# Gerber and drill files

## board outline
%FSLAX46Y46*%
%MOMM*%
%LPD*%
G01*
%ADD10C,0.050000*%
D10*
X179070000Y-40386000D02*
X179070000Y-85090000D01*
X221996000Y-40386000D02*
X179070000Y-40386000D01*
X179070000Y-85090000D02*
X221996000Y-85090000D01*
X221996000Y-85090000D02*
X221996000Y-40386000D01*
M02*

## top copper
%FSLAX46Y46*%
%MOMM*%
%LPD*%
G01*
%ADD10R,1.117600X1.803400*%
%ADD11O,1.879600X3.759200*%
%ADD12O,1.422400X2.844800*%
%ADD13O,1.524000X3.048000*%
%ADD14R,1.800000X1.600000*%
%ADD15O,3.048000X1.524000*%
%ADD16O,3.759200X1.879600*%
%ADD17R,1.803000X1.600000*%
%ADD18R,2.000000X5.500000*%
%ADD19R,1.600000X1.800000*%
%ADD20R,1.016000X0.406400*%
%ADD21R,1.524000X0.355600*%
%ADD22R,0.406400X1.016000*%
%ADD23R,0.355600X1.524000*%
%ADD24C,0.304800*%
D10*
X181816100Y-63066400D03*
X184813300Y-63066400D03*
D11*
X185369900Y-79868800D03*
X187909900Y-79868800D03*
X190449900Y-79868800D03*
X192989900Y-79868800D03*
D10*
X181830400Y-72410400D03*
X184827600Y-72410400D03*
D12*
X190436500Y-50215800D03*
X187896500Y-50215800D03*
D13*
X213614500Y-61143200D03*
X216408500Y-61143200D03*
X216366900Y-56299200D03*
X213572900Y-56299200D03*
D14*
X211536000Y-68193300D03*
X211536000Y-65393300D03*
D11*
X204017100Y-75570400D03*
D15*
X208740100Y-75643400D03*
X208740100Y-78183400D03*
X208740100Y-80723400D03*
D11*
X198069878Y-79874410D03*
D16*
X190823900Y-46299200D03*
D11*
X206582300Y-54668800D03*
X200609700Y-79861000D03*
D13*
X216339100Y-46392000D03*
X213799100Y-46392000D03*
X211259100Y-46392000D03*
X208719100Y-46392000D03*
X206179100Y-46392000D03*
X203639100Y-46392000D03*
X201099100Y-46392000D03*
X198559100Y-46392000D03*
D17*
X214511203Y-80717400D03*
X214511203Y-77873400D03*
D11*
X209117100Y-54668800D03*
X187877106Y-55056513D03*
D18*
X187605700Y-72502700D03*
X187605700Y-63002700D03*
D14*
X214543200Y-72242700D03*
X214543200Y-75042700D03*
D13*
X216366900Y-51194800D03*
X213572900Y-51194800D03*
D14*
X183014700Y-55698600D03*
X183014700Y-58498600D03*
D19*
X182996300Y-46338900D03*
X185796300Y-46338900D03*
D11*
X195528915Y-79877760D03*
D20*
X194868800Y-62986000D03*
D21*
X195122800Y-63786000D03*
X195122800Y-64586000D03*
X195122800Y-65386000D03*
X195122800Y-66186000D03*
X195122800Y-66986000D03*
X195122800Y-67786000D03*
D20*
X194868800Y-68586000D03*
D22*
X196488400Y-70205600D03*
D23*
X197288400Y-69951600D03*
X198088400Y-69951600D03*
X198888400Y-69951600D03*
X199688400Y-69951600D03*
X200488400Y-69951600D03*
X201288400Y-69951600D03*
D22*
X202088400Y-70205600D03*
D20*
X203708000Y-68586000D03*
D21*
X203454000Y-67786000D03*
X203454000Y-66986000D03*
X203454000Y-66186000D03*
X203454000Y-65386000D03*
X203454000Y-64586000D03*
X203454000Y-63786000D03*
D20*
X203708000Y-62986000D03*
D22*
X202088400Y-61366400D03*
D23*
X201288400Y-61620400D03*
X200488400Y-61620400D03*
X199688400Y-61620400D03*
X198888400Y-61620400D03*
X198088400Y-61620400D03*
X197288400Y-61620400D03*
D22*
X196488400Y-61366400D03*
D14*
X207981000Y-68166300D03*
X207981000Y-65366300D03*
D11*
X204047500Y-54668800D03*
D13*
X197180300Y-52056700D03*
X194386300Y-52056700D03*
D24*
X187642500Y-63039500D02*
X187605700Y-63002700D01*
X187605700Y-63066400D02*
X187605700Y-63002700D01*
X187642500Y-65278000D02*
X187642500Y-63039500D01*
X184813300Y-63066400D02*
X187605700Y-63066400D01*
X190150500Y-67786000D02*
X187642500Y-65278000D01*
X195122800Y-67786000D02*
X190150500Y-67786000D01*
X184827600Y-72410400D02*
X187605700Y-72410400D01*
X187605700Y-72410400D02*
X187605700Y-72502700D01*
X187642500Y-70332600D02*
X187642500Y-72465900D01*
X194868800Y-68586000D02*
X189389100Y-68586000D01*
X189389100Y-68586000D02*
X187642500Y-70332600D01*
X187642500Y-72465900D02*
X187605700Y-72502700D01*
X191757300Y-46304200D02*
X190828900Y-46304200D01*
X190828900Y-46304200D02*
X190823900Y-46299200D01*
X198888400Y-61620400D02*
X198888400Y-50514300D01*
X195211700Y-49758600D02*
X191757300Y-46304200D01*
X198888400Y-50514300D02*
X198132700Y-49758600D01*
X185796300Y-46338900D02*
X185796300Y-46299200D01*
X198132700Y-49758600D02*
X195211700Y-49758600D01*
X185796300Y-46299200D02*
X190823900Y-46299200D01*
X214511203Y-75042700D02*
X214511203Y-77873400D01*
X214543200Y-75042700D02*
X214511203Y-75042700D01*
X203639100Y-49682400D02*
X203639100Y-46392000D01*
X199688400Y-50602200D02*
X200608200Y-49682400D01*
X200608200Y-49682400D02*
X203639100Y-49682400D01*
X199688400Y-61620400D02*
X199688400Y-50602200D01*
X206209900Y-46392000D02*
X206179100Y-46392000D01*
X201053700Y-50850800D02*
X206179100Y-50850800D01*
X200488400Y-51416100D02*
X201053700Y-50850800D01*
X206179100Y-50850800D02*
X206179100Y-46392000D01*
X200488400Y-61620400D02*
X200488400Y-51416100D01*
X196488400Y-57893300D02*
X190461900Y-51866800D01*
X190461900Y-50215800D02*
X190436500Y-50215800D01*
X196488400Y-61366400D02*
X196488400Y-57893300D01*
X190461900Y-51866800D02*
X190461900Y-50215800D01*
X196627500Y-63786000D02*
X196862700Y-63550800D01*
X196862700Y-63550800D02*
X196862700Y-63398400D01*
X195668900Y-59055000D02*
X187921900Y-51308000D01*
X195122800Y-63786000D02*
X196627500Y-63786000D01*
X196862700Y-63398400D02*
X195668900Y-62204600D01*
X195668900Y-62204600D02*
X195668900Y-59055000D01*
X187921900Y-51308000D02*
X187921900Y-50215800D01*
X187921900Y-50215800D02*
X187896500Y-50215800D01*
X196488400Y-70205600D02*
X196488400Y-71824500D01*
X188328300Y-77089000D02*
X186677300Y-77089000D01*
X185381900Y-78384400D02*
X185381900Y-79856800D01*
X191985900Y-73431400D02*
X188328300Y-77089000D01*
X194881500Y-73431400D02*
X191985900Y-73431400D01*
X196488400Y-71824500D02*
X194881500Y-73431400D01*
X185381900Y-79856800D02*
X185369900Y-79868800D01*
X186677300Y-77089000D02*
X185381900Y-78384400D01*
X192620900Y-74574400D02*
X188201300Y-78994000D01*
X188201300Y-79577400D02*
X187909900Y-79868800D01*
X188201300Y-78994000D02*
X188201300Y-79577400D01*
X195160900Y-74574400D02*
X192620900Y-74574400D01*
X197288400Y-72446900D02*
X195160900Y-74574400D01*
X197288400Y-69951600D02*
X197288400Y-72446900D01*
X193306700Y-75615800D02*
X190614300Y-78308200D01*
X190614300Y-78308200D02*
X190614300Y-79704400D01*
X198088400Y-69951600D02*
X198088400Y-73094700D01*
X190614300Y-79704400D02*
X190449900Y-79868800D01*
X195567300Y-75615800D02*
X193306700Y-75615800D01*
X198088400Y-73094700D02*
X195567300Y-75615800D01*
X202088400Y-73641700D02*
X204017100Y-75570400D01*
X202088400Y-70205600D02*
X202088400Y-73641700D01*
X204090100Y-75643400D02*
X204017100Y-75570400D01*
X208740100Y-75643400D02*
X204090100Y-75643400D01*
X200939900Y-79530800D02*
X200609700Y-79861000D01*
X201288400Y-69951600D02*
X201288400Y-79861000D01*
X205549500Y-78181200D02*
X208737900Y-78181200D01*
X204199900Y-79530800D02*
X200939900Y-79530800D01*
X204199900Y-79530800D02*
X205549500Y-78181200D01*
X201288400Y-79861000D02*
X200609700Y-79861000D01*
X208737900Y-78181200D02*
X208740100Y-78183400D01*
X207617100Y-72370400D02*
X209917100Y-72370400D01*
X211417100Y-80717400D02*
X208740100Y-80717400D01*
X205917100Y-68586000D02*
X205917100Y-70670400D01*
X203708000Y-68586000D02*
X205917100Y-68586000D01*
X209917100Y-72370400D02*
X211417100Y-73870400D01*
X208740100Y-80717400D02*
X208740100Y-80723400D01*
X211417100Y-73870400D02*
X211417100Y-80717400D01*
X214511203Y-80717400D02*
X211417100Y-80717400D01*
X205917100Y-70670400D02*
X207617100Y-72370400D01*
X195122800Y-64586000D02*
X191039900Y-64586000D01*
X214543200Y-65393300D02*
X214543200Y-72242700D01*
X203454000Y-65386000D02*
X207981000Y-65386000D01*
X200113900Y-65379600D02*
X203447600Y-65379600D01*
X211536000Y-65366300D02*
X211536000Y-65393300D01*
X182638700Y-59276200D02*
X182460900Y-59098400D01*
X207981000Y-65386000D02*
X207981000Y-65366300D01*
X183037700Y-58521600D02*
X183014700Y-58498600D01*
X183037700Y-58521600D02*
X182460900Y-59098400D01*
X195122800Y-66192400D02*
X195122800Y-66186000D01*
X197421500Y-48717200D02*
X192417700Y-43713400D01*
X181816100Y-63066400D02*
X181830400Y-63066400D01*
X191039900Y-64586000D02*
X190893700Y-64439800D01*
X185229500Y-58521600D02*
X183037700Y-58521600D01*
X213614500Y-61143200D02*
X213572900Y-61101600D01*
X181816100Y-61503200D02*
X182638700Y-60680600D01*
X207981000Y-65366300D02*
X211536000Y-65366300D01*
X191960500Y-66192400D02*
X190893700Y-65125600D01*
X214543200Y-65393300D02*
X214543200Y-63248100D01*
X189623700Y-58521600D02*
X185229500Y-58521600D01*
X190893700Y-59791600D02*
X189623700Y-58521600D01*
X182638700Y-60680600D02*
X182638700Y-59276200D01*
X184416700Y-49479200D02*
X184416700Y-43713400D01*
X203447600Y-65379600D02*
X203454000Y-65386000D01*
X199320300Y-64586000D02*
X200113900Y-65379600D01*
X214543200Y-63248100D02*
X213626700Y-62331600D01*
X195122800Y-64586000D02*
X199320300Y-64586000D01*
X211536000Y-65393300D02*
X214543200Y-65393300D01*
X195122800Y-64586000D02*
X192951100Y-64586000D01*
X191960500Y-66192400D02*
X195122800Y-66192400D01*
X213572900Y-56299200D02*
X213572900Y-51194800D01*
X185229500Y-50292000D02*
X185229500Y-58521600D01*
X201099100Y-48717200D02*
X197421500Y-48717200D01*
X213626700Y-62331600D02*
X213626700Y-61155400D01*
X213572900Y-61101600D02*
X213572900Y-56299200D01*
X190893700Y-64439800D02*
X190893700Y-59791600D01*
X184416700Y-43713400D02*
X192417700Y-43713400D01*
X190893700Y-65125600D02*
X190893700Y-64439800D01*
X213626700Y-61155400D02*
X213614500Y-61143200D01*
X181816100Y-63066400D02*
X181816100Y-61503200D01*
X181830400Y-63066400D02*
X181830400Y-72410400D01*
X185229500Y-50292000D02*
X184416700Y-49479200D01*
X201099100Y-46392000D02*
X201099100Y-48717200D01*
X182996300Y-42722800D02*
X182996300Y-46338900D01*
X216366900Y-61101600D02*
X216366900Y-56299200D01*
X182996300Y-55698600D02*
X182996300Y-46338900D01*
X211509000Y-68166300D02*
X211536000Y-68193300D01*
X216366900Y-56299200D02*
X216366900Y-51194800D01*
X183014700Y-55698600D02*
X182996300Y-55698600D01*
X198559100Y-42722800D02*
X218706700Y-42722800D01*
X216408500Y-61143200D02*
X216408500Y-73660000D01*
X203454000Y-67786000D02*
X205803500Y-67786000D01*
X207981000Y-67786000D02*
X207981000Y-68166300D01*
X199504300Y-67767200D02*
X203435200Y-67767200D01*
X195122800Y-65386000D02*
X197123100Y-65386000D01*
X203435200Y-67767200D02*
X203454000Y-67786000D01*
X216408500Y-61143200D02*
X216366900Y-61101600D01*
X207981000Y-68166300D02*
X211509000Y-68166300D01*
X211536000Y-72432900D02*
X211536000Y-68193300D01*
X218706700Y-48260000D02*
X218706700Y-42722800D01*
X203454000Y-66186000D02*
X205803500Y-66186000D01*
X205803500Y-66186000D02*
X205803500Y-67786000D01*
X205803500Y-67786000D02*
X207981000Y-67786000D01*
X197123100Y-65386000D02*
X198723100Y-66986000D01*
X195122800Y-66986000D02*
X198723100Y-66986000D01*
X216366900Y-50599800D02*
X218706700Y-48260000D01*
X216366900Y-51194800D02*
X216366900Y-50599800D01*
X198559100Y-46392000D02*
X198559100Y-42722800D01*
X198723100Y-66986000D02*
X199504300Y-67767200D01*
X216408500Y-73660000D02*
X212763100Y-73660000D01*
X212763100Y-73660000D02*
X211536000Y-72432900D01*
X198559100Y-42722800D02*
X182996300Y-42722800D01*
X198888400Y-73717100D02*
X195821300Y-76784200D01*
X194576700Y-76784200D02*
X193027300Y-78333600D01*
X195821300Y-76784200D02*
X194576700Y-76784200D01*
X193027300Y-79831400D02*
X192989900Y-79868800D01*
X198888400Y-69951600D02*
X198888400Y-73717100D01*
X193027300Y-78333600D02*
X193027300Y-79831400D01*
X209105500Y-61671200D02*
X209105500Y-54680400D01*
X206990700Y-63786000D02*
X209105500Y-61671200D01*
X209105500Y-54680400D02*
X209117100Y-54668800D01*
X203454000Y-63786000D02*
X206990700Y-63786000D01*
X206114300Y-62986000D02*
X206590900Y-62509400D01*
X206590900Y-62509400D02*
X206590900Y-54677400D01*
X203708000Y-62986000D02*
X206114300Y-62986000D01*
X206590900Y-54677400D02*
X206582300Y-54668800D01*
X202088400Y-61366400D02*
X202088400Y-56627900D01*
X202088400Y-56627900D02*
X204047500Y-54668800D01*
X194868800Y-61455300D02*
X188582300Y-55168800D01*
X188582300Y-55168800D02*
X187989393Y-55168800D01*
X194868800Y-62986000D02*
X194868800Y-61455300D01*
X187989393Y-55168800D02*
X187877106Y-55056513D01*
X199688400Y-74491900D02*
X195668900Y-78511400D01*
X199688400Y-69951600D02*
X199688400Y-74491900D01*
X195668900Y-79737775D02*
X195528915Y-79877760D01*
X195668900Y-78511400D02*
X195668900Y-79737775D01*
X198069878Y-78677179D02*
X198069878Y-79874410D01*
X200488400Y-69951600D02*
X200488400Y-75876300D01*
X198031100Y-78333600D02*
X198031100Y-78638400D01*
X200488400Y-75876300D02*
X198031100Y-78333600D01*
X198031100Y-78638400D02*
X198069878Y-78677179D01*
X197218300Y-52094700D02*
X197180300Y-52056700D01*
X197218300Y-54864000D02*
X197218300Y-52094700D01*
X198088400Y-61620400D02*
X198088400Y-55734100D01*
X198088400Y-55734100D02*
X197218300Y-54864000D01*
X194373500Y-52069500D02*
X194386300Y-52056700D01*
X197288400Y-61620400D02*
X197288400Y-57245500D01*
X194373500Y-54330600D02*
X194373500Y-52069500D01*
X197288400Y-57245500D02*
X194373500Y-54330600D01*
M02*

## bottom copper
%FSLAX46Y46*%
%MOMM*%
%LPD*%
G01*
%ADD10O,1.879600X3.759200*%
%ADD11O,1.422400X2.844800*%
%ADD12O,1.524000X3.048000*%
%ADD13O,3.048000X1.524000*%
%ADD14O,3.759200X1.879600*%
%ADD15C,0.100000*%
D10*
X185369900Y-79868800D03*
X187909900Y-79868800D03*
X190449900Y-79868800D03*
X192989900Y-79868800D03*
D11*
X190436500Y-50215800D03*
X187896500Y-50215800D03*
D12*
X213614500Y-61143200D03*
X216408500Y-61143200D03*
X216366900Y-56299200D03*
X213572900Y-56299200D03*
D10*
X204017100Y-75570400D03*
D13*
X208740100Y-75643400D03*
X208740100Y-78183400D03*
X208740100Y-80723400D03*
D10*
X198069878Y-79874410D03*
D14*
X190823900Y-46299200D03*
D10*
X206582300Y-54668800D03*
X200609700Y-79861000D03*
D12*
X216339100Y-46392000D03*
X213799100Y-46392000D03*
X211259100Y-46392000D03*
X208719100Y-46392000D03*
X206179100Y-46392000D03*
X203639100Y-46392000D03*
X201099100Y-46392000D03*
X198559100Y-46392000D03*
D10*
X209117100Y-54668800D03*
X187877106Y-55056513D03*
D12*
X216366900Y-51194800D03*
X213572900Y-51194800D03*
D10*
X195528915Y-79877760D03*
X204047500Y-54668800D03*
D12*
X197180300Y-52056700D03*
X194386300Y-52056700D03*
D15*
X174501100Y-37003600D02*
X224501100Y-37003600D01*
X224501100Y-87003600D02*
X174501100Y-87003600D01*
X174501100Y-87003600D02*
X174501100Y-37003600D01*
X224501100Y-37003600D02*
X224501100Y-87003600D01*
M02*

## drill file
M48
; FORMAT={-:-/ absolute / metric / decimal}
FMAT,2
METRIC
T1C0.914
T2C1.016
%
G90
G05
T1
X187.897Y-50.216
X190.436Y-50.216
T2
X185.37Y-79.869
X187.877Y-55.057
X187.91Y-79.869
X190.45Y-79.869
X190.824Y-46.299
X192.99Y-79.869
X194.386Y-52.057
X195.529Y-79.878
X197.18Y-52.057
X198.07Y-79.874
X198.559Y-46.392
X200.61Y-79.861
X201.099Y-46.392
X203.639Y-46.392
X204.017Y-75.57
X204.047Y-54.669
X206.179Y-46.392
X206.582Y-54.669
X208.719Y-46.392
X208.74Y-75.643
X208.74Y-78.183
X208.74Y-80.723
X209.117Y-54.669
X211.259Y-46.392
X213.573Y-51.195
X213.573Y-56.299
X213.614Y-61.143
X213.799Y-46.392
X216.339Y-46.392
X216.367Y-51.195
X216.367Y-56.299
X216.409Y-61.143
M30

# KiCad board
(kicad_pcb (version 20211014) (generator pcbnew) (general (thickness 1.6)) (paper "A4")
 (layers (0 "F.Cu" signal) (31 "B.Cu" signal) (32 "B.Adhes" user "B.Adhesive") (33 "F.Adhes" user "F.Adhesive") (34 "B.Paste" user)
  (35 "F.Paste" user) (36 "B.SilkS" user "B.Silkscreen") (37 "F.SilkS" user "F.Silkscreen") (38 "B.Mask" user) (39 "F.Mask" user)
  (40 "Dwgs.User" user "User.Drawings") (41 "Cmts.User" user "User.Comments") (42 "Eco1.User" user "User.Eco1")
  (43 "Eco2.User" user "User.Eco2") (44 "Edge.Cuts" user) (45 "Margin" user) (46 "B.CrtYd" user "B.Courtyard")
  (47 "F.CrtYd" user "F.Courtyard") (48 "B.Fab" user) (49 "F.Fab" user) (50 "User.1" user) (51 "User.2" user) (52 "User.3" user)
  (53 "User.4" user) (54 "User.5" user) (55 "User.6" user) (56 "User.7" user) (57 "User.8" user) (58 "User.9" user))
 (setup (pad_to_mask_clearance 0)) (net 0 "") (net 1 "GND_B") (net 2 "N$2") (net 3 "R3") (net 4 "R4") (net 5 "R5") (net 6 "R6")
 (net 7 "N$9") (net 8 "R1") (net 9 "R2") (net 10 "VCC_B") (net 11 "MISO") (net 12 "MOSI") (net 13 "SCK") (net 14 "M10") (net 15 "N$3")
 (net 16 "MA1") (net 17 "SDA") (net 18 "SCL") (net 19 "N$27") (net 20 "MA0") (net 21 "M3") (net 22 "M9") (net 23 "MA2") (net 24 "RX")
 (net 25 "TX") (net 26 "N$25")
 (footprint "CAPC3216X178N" (layer "F.Cu") (at 183.3147 63.0664)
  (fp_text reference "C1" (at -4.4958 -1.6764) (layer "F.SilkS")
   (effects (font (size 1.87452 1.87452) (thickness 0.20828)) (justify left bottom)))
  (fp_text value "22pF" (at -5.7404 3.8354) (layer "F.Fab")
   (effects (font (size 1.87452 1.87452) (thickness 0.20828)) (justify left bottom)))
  (pad "1" smd rect (at -1.4986 0) (size 1.1176 1.8034) (layers "F.Cu" "F.Paste" "F.Mask") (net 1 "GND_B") (solder_mask_margin 0.1016))
  (pad "2" smd rect (at 1.4986 0) (size 1.1176 1.8034) (layers "F.Cu" "F.Paste" "F.Mask") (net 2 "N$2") (solder_mask_margin 0.1016)))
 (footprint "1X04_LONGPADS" (layer "F.Cu") (at 185.3699 79.8688)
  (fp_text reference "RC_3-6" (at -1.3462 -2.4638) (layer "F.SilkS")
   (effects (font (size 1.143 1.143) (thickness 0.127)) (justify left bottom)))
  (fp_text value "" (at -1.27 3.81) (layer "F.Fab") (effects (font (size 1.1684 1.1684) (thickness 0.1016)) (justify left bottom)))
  (pad "1" thru_hole oval (at 0 0 90) (size 3.7592 1.8796) (drill 1.016) (layers *.Cu *.Mask) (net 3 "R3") (solder_mask_margin 0.1016))
  (pad "2" thru_hole oval (at 2.54 0 90) (size 3.7592 1.8796) (drill 1.016) (layers *.Cu *.Mask) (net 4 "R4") (solder_mask_margin 0.1016))
  (pad "3" thru_hole oval (at 5.08 0 90) (size 3.7592 1.8796) (drill 1.016) (layers *.Cu *.Mask) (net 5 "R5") (solder_mask_margin 0.1016))
  (pad "4" thru_hole oval (at 7.62 0 90) (size 3.7592 1.8796) (drill 1.016) (layers *.Cu *.Mask) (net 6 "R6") (solder_mask_margin 0.1016)))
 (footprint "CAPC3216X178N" (layer "F.Cu") (at 183.329 72.4104)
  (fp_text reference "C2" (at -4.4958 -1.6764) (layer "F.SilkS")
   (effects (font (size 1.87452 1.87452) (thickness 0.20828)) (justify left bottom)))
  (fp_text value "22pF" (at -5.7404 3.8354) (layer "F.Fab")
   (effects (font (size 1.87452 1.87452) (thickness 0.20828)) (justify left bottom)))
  (pad "1" smd rect (at -1.4986 0) (size 1.1176 1.8034) (layers "F.Cu" "F.Paste" "F.Mask") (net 1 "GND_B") (solder_mask_margin 0.1016))
  (pad "2" smd rect (at 1.4986 0) (size 1.1176 1.8034) (layers "F.Cu" "F.Paste" "F.Mask") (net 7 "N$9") (solder_mask_margin 0.1016)))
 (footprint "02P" (layer "F.Cu") (at 189.1665 50.2158 180)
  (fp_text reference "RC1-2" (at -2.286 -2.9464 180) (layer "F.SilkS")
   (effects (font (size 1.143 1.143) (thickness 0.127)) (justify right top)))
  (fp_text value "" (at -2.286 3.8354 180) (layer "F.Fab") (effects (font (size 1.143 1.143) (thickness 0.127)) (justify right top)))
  (pad "1" thru_hole oval (at -1.27 0 270) (size 2.8448 1.4224) (drill 0.9144) (layers *.Cu *.Mask) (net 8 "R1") (solder_mask_margin 0.1016))
  (pad "2" thru_hole oval (at 1.27 0 270) (size 2.8448 1.4224) (drill 0.9144) (layers *.Cu *.Mask) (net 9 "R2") (solder_mask_margin 0.1016)))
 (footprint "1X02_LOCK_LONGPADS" (layer "F.Cu") (at 213.7415 61.1432)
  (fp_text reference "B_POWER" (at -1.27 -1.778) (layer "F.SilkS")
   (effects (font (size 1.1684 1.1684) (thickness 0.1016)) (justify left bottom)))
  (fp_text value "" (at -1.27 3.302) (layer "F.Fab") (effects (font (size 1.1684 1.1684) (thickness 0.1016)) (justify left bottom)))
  (pad "1" thru_hole oval (at -0.127 0 90) (size 3.048 1.524) (drill 1.016) (layers *.Cu *.Mask) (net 1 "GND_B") (solder_mask_margin 0.1016))
  (pad "2" thru_hole oval (at 2.667 0 90) (size 3.048 1.524) (drill 1.016) (layers *.Cu *.Mask) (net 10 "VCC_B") (solder_mask_margin 0.1016)))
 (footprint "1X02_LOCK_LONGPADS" (layer "F.Cu") (at 216.2399 56.2992 180)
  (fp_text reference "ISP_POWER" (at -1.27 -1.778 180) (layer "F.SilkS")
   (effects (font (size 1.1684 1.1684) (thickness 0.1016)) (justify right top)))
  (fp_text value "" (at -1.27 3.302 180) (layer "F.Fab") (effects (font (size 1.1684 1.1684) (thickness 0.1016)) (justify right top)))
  (pad "1" thru_hole oval (at -0.127 0 270) (size 3.048 1.524) (drill 1.016) (layers *.Cu *.Mask) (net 10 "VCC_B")
   (solder_mask_margin 0.1016))
  (pad "2" thru_hole oval (at 2.667 0 270) (size 3.048 1.524) (drill 1.016) (layers *.Cu *.Mask) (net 1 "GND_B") (solder_mask_margin 0.1016)))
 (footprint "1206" (layer "F.Cu") (at 211.536 66.7933 90)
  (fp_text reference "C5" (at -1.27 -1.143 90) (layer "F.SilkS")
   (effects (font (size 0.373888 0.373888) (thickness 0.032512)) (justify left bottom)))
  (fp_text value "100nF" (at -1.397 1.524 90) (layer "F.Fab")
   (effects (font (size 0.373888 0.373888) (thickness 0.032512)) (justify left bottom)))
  (pad "1" smd rect (at -1.4 0 90) (size 1.6 1.8) (layers "F.Cu" "F.Paste" "F.Mask") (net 10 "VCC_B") (solder_mask_margin 0.1016))
  (pad "2" smd rect (at 1.4 0 90) (size 1.6 1.8) (layers "F.Cu" "F.Paste" "F.Mask") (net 1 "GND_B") (solder_mask_margin 0.1016)))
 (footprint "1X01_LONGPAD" (layer "F.Cu") (at 204.0171 75.5704)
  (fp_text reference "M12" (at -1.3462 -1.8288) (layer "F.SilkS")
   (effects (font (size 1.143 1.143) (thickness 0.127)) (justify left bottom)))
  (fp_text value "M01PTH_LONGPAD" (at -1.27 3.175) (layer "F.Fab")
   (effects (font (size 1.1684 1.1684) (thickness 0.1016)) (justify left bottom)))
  (pad "1" thru_hole oval (at 0 0 90) (size 3.7592 1.8796) (drill 1.016) (layers *.Cu *.Mask) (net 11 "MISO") (solder_mask_margin 0.1016)))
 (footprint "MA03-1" (layer "F.Cu") (at 208.7401 78.1834 -90)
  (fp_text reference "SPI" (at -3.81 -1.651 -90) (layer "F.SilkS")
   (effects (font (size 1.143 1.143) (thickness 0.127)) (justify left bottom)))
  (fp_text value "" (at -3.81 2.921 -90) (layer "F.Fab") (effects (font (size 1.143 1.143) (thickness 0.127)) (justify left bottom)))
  (pad "1" thru_hole oval (at -2.54 0) (size 3.048 1.524) (drill 1.016) (layers *.Cu *.Mask) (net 11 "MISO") (solder_mask_margin 0.1016))
  (pad "2" thru_hole oval (at 0 0) (size 3.048 1.524) (drill 1.016) (layers *.Cu *.Mask) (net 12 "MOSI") (solder_mask_margin 0.1016))
  (pad "3" thru_hole oval (at 2.54 0) (size 3.048 1.524) (drill 1.016) (layers *.Cu *.Mask) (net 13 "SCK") (solder_mask_margin 0.1016)))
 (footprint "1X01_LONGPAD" (layer "F.Cu") (at 198.069878 79.87441)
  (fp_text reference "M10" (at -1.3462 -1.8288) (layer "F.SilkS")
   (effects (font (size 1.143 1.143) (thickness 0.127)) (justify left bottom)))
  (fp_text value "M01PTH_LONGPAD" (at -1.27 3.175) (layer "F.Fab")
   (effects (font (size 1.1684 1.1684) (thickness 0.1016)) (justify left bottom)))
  (pad "1" thru_hole oval (at 0 0 90) (size 3.7592 1.8796) (drill 1.016) (layers *.Cu *.Mask) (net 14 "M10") (solder_mask_margin 0.1016)))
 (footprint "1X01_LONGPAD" (layer "F.Cu") (at 190.8239 46.2992 90)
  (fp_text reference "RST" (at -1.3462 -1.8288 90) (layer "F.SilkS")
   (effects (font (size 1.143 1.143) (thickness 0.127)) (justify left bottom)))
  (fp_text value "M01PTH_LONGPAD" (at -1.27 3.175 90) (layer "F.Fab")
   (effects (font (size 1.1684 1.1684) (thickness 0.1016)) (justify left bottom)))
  (pad "1" thru_hole oval (at 0 0 180) (size 3.7592 1.8796) (drill 1.016) (layers *.Cu *.Mask) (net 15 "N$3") (solder_mask_margin 0.1016)))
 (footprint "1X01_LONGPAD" (layer "F.Cu") (at 206.5823 54.6688 180)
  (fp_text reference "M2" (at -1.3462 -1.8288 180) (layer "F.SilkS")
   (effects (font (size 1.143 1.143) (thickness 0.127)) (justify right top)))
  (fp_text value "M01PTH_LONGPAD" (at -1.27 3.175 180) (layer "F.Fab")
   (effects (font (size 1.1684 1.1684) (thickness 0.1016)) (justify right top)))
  (pad "1" thru_hole oval (at 0 0 270) (size 3.7592 1.8796) (drill 1.016) (layers *.Cu *.Mask) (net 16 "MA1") (solder_mask_margin 0.1016)))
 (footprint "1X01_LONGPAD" (layer "F.Cu") (at 200.6097 79.861 180)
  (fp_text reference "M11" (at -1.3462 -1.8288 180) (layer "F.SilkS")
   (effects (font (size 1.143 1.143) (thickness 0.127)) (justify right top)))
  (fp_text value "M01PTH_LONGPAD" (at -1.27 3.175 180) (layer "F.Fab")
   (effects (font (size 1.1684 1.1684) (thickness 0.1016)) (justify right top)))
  (pad "1" thru_hole oval (at 0 0 270) (size 3.7592 1.8796) (drill 1.016) (layers *.Cu *.Mask) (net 12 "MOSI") (solder_mask_margin 0.1016)))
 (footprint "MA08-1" (layer "F.Cu") (at 207.4491 46.392 180)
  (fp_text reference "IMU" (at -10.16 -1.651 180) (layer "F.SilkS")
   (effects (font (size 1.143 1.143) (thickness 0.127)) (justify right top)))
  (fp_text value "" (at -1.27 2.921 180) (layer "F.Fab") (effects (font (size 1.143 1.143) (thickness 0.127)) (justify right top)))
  (pad "1" thru_hole oval (at -8.89 0 270) (size 3.048 1.524) (drill 1.016) (layers *.Cu *.Mask) (solder_mask_margin 0.1016))
  (pad "2" thru_hole oval (at -6.35 0 270) (size 3.048 1.524) (drill 1.016) (layers *.Cu *.Mask) (solder_mask_margin 0.1016))
  (pad "3" thru_hole oval (at -3.81 0 270) (size 3.048 1.524) (drill 1.016) (layers *.Cu *.Mask) (solder_mask_margin 0.1016))
  (pad "4" thru_hole oval (at -1.27 0 270) (size 3.048 1.524) (drill 1.016) (layers *.Cu *.Mask) (solder_mask_margin 0.1016))
  (pad "5" thru_hole oval (at 1.27 0 270) (size 3.048 1.524) (drill 1.016) (layers *.Cu *.Mask) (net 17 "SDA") (solder_mask_margin 0.1016))
  (pad "6" thru_hole oval (at 3.81 0 270) (size 3.048 1.524) (drill 1.016) (layers *.Cu *.Mask) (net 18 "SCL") (solder_mask_margin 0.1016))
  (pad "7" thru_hole oval (at 6.35 0 270) (size 3.048 1.524) (drill 1.016) (layers *.Cu *.Mask) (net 1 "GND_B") (solder_mask_margin 0.1016))
  (pad "8" thru_hole oval (at 8.89 0 270) (size 3.048 1.524) (drill 1.016) (layers *.Cu *.Mask) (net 10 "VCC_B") (solder_mask_margin 0.1016)))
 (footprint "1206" (layer "F.Cu") (at 214.511203 79.2954 90)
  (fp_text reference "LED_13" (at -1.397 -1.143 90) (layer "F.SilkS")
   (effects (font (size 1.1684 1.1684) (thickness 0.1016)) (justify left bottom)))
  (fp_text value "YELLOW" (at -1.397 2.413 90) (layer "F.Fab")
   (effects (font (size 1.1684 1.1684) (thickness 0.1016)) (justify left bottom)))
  (pad "1" smd rect (at -1.422 0 90) (size 1.6 1.803) (layers "F.Cu" "F.Paste" "F.Mask") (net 13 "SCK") (solder_mask_margin 0.1016))
  (pad "2" smd rect (at 1.422 0 90) (size 1.6 1.803) (layers "F.Cu" "F.Paste" "F.Mask") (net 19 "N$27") (solder_mask_margin 0.1016)))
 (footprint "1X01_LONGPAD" (layer "F.Cu") (at 209.1171 54.6688 180)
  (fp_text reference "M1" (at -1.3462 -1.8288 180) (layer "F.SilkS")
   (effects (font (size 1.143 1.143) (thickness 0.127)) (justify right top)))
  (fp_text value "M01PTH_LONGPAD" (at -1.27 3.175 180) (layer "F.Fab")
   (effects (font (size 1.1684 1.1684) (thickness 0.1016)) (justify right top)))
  (pad "1" thru_hole oval (at 0 0 270) (size 3.7592 1.8796) (drill 1.016) (layers *.Cu *.Mask) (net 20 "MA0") (solder_mask_margin 0.1016)))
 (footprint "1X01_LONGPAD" (layer "F.Cu") (at 187.877106 55.056513 180)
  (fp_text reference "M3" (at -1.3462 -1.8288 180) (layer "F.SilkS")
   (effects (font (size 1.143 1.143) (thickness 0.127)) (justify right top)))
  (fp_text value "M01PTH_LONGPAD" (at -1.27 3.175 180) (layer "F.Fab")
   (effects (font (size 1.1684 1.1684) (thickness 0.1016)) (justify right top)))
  (pad "1" thru_hole oval (at 0 0 270) (size 3.7592 1.8796) (drill 1.016) (layers *.Cu *.Mask) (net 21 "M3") (solder_mask_margin 0.1016)))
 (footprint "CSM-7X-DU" (layer "F.Cu") (at 187.6057 67.7527 90)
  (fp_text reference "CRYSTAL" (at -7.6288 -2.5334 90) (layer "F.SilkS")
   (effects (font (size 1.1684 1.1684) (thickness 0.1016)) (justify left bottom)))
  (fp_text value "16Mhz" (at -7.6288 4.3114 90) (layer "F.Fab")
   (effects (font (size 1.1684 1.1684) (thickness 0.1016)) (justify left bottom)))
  (pad "1" smd rect (at -4.75 0 90) (size 5.5 2) (layers "F.Cu" "F.Paste" "F.Mask") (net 7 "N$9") (solder_mask_margin 0.1016))
  (pad "2" smd rect (at 4.75 0 90) (size 5.5 2) (layers "F.Cu" "F.Paste" "F.Mask") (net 2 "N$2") (solder_mask_margin 0.1016)))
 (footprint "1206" (layer "F.Cu") (at 214.5432 73.6427 -90)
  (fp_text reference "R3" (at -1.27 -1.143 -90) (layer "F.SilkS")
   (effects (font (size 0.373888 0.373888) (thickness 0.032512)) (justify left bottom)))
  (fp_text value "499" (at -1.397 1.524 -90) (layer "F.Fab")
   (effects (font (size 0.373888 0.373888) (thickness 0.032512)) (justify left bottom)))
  (pad "1" smd rect (at -1.4 0 270) (size 1.6 1.8) (layers "F.Cu" "F.Paste" "F.Mask") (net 1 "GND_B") (solder_mask_margin 0.1016))
  (pad "2" smd rect (at 1.4 0 270) (size 1.6 1.8) (layers "F.Cu" "F.Paste" "F.Mask") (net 19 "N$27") (solder_mask_margin 0.1016)))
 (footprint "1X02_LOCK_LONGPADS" (layer "F.Cu") (at 216.2399 51.1948 180)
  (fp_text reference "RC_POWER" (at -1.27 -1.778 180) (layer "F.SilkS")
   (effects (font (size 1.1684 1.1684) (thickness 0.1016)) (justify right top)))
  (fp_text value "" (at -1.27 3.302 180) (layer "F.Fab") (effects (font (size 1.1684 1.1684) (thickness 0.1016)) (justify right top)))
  (pad "1" thru_hole oval (at -0.127 0 270) (size 3.048 1.524) (drill 1.016) (layers *.Cu *.Mask) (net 10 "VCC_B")
   (solder_mask_margin 0.1016))
  (pad "2" thru_hole oval (at 2.667 0 270) (size 3.048 1.524) (drill 1.016) (layers *.Cu *.Mask) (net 1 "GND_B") (solder_mask_margin 0.1016)))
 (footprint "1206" (layer "F.Cu") (at 183.0147 57.0986 -90)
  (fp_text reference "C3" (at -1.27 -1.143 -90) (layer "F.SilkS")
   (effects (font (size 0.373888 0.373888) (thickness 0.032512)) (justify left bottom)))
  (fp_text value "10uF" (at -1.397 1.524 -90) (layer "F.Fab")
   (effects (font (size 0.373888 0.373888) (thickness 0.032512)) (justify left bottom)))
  (pad "1" smd rect (at -1.4 0 270) (size 1.6 1.8) (layers "F.Cu" "F.Paste" "F.Mask") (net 10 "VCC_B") (solder_mask_margin 0.1016))
  (pad "2" smd rect (at 1.4 0 270) (size 1.6 1.8) (layers "F.Cu" "F.Paste" "F.Mask") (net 1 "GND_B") (solder_mask_margin 0.1016)))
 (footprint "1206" (layer "F.Cu") (at 184.3963 46.3389)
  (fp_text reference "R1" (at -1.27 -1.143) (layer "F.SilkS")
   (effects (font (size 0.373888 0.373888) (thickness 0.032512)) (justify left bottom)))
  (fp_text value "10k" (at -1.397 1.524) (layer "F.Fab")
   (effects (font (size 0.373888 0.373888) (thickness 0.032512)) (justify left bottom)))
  (pad "1" smd rect (at -1.4 0) (size 1.6 1.8) (layers "F.Cu" "F.Paste" "F.Mask") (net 10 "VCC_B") (solder_mask_margin 0.1016))
  (pad "2" smd rect (at 1.4 0) (size 1.6 1.8) (layers "F.Cu" "F.Paste" "F.Mask") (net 15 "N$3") (solder_mask_margin 0.1016)))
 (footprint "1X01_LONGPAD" (layer "F.Cu") (at 195.528915 79.87776)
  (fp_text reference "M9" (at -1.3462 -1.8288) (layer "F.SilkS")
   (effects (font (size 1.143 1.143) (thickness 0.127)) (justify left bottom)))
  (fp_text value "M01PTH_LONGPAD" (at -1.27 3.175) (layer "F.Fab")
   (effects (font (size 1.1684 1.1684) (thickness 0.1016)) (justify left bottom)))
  (pad "1" thru_hole oval (at 0 0 90) (size 3.7592 1.8796) (drill 1.016) (layers *.Cu *.Mask) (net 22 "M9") (solder_mask_margin 0.1016)))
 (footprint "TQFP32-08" (layer "F.Cu") (at 199.2884 65.786)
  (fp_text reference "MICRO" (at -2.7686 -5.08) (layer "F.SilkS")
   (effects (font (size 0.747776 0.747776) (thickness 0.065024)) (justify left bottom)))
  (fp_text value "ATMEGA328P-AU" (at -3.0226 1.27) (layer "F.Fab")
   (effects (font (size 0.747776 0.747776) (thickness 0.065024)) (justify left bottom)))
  (pad "1" smd rect (at -4.4196 -2.8) (size 1.016 0.4064) (layers "F.Cu" "F.Paste" "F.Mask") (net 21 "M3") (solder_mask_margin 0.1016))
  (pad "2" smd rect (at -4.1656 -2) (size 1.524 0.3556) (layers "F.Cu" "F.Paste" "F.Mask") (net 9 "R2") (solder_mask_margin 0.1016))
  (pad "3" smd rect (at -4.1656 -1.2) (size 1.524 0.3556) (layers "F.Cu" "F.Paste" "F.Mask") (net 1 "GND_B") (solder_mask_margin 0.1016))
  (pad "4" smd rect (at -4.1656 -0.4) (size 1.524 0.3556) (layers "F.Cu" "F.Paste" "F.Mask") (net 10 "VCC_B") (solder_mask_margin 0.1016))
  (pad "5" smd rect (at -4.1656 0.4) (size 1.524 0.3556) (layers "F.Cu" "F.Paste" "F.Mask") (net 1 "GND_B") (solder_mask_margin 0.1016))
  (pad "6" smd rect (at -4.1656 1.2) (size 1.524 0.3556) (layers "F.Cu" "F.Paste" "F.Mask") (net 10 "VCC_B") (solder_mask_margin 0.1016))
  (pad "7" smd rect (at -4.1656 2) (size 1.524 0.3556) (layers "F.Cu" "F.Paste" "F.Mask") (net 2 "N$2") (solder_mask_margin 0.1016))
  (pad "8" smd rect (at -4.4196 2.8) (size 1.016 0.4064) (layers "F.Cu" "F.Paste" "F.Mask") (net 7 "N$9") (solder_mask_margin 0.1016))
  (pad "9" smd rect (at -2.8 4.4196) (size 0.4064 1.016) (layers "F.Cu" "F.Paste" "F.Mask") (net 3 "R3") (solder_mask_margin 0.1016))
  (pad "10" smd rect (at -2 4.1656) (size 0.3556 1.524) (layers "F.Cu" "F.Paste" "F.Mask") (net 4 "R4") (solder_mask_margin 0.1016))
  (pad "11" smd rect (at -1.2 4.1656) (size 0.3556 1.524) (layers "F.Cu" "F.Paste" "F.Mask") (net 5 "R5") (solder_mask_margin 0.1016))
  (pad "12" smd rect (at -0.4 4.1656) (size 0.3556 1.524) (layers "F.Cu" "F.Paste" "F.Mask") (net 6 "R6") (solder_mask_margin 0.1016))
  (pad "13" smd rect (at 0.4 4.1656) (size 0.3556 1.524) (layers "F.Cu" "F.Paste" "F.Mask") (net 22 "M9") (solder_mask_margin 0.1016))
  (pad "14" smd rect (at 1.2 4.1656) (size 0.3556 1.524) (layers "F.Cu" "F.Paste" "F.Mask") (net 14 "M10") (solder_mask_margin 0.1016))
  (pad "15" smd rect (at 2 4.1656) (size 0.3556 1.524) (layers "F.Cu" "F.Paste" "F.Mask") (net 12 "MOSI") (solder_mask_margin 0.1016))
  (pad "16" smd rect (at 2.8 4.4196) (size 0.4064 1.016) (layers "F.Cu" "F.Paste" "F.Mask") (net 11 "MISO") (solder_mask_margin 0.1016))
  (pad "17" smd rect (at 4.4196 2.8) (size 1.016 0.4064) (layers "F.Cu" "F.Paste" "F.Mask") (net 13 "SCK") (solder_mask_margin 0.1016))
  (pad "18" smd rect (at 4.1656 2) (size 1.524 0.3556) (layers "F.Cu" "F.Paste" "F.Mask") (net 10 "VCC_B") (solder_mask_margin 0.1016))
  (pad "19" smd rect (at 4.1656 1.2) (size 1.524 0.3556) (layers "F.Cu" "F.Paste" "F.Mask") (solder_mask_margin 0.1016))
  (pad "20" smd rect (at 4.1656 0.4) (size 1.524 0.3556) (layers "F.Cu" "F.Paste" "F.Mask") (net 10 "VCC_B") (solder_mask_margin 0.1016))
  (pad "21" smd rect (at 4.1656 -0.4) (size 1.524 0.3556) (layers "F.Cu" "F.Paste" "F.Mask") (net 1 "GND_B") (solder_mask_margin 0.1016))
  (pad "22" smd rect (at 4.1656 -1.2) (size 1.524 0.3556) (layers "F.Cu" "F.Paste" "F.Mask") (solder_mask_margin 0.1016))
  (pad "23" smd rect (at 4.1656 -2) (size 1.524 0.3556) (layers "F.Cu" "F.Paste" "F.Mask") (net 20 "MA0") (solder_mask_margin 0.1016))
  (pad "24" smd rect (at 4.4196 -2.8) (size 1.016 0.4064) (layers "F.Cu" "F.Paste" "F.Mask") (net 16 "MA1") (solder_mask_margin 0.1016))
  (pad "25" smd rect (at 2.8 -4.4196) (size 0.4064 1.016) (layers "F.Cu" "F.Paste" "F.Mask") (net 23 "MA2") (solder_mask_margin 0.1016))
  (pad "26" smd rect (at 2 -4.1656) (size 0.3556 1.524) (layers "F.Cu" "F.Paste" "F.Mask") (solder_mask_margin 0.1016))
  (pad "27" smd rect (at 1.2 -4.1656) (size 0.3556 1.524) (layers "F.Cu" "F.Paste" "F.Mask") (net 17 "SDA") (solder_mask_margin 0.1016))
  (pad "28" smd rect (at 0.4 -4.1656) (size 0.3556 1.524) (layers "F.Cu" "F.Paste" "F.Mask") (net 18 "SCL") (solder_mask_margin 0.1016))
  (pad "29" smd rect (at -0.4 -4.1656) (size 0.3556 1.524) (layers "F.Cu" "F.Paste" "F.Mask") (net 15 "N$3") (solder_mask_margin 0.1016))
  (pad "30" smd rect (at -1.2 -4.1656) (size 0.3556 1.524) (layers "F.Cu" "F.Paste" "F.Mask") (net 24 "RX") (solder_mask_margin 0.1016))
  (pad "31" smd rect (at -2 -4.1656) (size 0.3556 1.524) (layers "F.Cu" "F.Paste" "F.Mask") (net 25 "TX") (solder_mask_margin 0.1016))
  (pad "32" smd rect (at -2.8 -4.4196) (size 0.4064 1.016) (layers "F.Cu" "F.Paste" "F.Mask") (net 8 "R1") (solder_mask_margin 0.1016)))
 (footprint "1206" (layer "F.Cu") (at 207.981 66.7663 90)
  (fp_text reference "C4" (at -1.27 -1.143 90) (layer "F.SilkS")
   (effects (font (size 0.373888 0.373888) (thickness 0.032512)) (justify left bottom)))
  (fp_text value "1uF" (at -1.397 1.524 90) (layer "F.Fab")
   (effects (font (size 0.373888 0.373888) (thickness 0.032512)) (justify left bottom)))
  (pad "1" smd rect (at -1.4 0 90) (size 1.6 1.8) (layers "F.Cu" "F.Paste" "F.Mask") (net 10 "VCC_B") (solder_mask_margin 0.1016))
  (pad "2" smd rect (at 1.4 0 90) (size 1.6 1.8) (layers "F.Cu" "F.Paste" "F.Mask") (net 1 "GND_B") (solder_mask_margin 0.1016)))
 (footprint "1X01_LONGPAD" (layer "F.Cu") (at 204.0475 54.6688 180)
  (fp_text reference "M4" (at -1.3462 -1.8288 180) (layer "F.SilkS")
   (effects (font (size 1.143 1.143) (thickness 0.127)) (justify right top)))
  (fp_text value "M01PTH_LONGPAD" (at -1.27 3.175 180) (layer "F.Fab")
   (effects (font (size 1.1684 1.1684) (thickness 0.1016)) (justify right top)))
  (pad "1" thru_hole oval (at 0 0 270) (size 3.7592 1.8796) (drill 1.016) (layers *.Cu *.Mask) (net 23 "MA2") (solder_mask_margin 0.1016)))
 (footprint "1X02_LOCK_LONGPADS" (layer "F.Cu") (at 197.0533 52.0567 180)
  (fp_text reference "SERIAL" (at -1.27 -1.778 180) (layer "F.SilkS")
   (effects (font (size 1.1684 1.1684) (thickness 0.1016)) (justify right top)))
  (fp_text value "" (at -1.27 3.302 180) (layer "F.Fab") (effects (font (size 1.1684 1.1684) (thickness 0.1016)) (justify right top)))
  (pad "1" thru_hole oval (at -0.127 0 270) (size 3.048 1.524) (drill 1.016) (layers *.Cu *.Mask) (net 24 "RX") (solder_mask_margin 0.1016))
  (pad "2" thru_hole oval (at 2.667 0 270) (size 3.048 1.524) (drill 1.016) (layers *.Cu *.Mask) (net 25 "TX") (solder_mask_margin 0.1016)))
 (gr_line (start 179.07 40.386) (end 179.07 85.09) (layer "Edge.Cuts") (width 0.05))
 (gr_line (start 221.996 40.386) (end 179.07 40.386) (layer "Edge.Cuts") (width 0.05))
 (gr_line (start 179.07 85.09) (end 221.996 85.09) (layer "Edge.Cuts") (width 0.05))
 (gr_line (start 221.996 85.09) (end 221.996 40.386) (layer "Edge.Cuts") (width 0.05))
 (segment (start 187.6425 63.0395) (end 187.6057 63.0027) (width 0.3048) (layer "F.Cu") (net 2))
 (segment (start 187.6057 63.0664) (end 187.6057 63.0027) (width 0.3048) (layer "F.Cu") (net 2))
 (segment (start 187.6425 65.278) (end 187.6425 63.0395) (width 0.3048) (layer "F.Cu") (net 2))
 (segment (start 184.8133 63.0664) (end 187.6057 63.0664) (width 0.3048) (layer "F.Cu") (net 2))
 (segment (start 190.1505 67.786) (end 187.6425 65.278) (width 0.3048) (layer "F.Cu") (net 2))
 (segment (start 195.1228 67.786) (end 190.1505 67.786) (width 0.3048) (layer "F.Cu") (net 2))
 (segment (start 184.8276 72.4104) (end 187.6057 72.4104) (width 0.3048) (layer "F.Cu") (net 7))
 (segment (start 187.6057 72.4104) (end 187.6057 72.5027) (width 0.3048) (layer "F.Cu") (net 7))
 (segment (start 187.6425 70.3326) (end 187.6425 72.4659) (width 0.3048) (layer "F.Cu") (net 7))
 (segment (start 194.8688 68.586) (end 189.3891 68.586) (width 0.3048) (layer "F.Cu") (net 7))
 (segment (start 189.3891 68.586) (end 187.6425 70.3326) (width 0.3048) (layer "F.Cu") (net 7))
 (segment (start 187.6425 72.4659) (end 187.6057 72.5027) (width 0.3048) (layer "F.Cu") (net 7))
 (segment (start 191.7573 46.3042) (end 190.8289 46.3042) (width 0.3048) (layer "F.Cu") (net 15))
 (segment (start 190.8289 46.3042) (end 190.8239 46.2992) (width 0.3048) (layer "F.Cu") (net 15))
 (segment (start 198.8884 61.6204) (end 198.8884 50.5143) (width 0.3048) (layer "F.Cu") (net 15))
 (segment (start 195.2117 49.7586) (end 191.7573 46.3042) (width 0.3048) (layer "F.Cu") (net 15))
 (segment (start 198.8884 50.5143) (end 198.1327 49.7586) (width 0.3048) (layer "F.Cu") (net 15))
 (segment (start 185.7963 46.3389) (end 185.7963 46.2992) (width 0.3048) (layer "F.Cu") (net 15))
 (segment (start 198.1327 49.7586) (end 195.2117 49.7586) (width 0.3048) (layer "F.Cu") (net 15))
 (segment (start 185.7963 46.2992) (end 190.8239 46.2992) (width 0.3048) (layer "F.Cu") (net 15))
 (segment (start 214.511203 75.0427) (end 214.511203 77.8734) (width 0.3048) (layer "F.Cu") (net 19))
 (segment (start 214.5432 75.0427) (end 214.511203 75.0427) (width 0.3048) (layer "F.Cu") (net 19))
 (segment (start 203.6391 49.6824) (end 203.6391 46.392) (width 0.3048) (layer "F.Cu") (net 18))
 (segment (start 199.6884 50.6022) (end 200.6082 49.6824) (width 0.3048) (layer "F.Cu") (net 18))
 (segment (start 200.6082 49.6824) (end 203.6391 49.6824) (width 0.3048) (layer "F.Cu") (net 18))
 (segment (start 199.6884 61.6204) (end 199.6884 50.6022) (width 0.3048) (layer "F.Cu") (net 18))
 (segment (start 206.2099 46.392) (end 206.1791 46.392) (width 0.3048) (layer "F.Cu") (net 17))
 (segment (start 201.0537 50.8508) (end 206.1791 50.8508) (width 0.3048) (layer "F.Cu") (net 17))
 (segment (start 200.4884 51.4161) (end 201.0537 50.8508) (width 0.3048) (layer "F.Cu") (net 17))
 (segment (start 206.1791 50.8508) (end 206.1791 46.392) (width 0.3048) (layer "F.Cu") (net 17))
 (segment (start 200.4884 61.6204) (end 200.4884 51.4161) (width 0.3048) (layer "F.Cu") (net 17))
 (segment (start 196.4884 57.8933) (end 190.4619 51.8668) (width 0.3048) (layer "F.Cu") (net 8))
 (segment (start 190.4619 50.2158) (end 190.4365 50.2158) (width 0.3048) (layer "F.Cu") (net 8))
 (segment (start 196.4884 61.3664) (end 196.4884 57.8933) (width 0.3048) (layer "F.Cu") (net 8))
 (segment (start 190.4619 51.8668) (end 190.4619 50.2158) (width 0.3048) (layer "F.Cu") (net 8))
 (segment (start 196.6275 63.786) (end 196.8627 63.5508) (width 0.3048) (layer "F.Cu") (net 9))
 (segment (start 196.8627 63.5508) (end 196.8627 63.3984) (width 0.3048) (layer "F.Cu") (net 9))
 (segment (start 195.6689 59.055) (end 187.9219 51.308) (width 0.3048) (layer "F.Cu") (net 9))
 (segment (start 195.1228 63.786) (end 196.6275 63.786) (width 0.3048) (layer "F.Cu") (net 9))
 (segment (start 196.8627 63.3984) (end 195.6689 62.2046) (width 0.3048) (layer "F.Cu") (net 9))
 (segment (start 195.6689 62.2046) (end 195.6689 59.055) (width 0.3048) (layer "F.Cu") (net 9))
 (segment (start 187.9219 51.308) (end 187.9219 50.2158) (width 0.3048) (layer "F.Cu") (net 9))
 (segment (start 187.9219 50.2158) (end 187.8965 50.2158) (width 0.3048) (layer "F.Cu") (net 9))
 (segment (start 196.4884 70.2056) (end 196.4884 71.8245) (width 0.3048) (layer "F.Cu") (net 3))
 (segment (start 188.3283 77.089) (end 186.6773 77.089) (width 0.3048) (layer "F.Cu") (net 3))
 (segment (start 185.3819 78.3844) (end 185.3819 79.8568) (width 0.3048) (layer "F.Cu") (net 3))
 (segment (start 191.9859 73.4314) (end 188.3283 77.089) (width 0.3048) (layer "F.Cu") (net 3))
 (segment (start 194.8815 73.4314) (end 191.9859 73.4314) (width 0.3048) (layer "F.Cu") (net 3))
 (segment (start 196.4884 71.8245) (end 194.8815 73.4314) (width 0.3048) (layer "F.Cu") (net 3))
 (segment (start 185.3819 79.8568) (end 185.3699 79.8688) (width 0.3048) (layer "F.Cu") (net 3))
 (segment (start 186.6773 77.089) (end 185.3819 78.3844) (width 0.3048) (layer "F.Cu") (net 3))
 (segment (start 192.6209 74.5744) (end 188.2013 78.994) (width 0.3048) (layer "F.Cu") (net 4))
 (segment (start 188.2013 79.5774) (end 187.9099 79.8688) (width 0.3048) (layer "F.Cu") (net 4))
 (segment (start 188.2013 78.994) (end 188.2013 79.5774) (width 0.3048) (layer "F.Cu") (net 4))
 (segment (start 195.1609 74.5744) (end 192.6209 74.5744) (width 0.3048) (layer "F.Cu") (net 4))
 (segment (start 197.2884 72.4469) (end 195.1609 74.5744) (width 0.3048) (layer "F.Cu") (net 4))
 (segment (start 197.2884 69.9516) (end 197.2884 72.4469) (width 0.3048) (layer "F.Cu") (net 4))
 (segment (start 193.3067 75.6158) (end 190.6143 78.3082) (width 0.3048) (layer "F.Cu") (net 5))
 (segment (start 190.6143 78.3082) (end 190.6143 79.7044) (width 0.3048) (layer "F.Cu") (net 5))
 (segment (start 198.0884 69.9516) (end 198.0884 73.0947) (width 0.3048) (layer "F.Cu") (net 5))
 (segment (start 190.6143 79.7044) (end 190.4499 79.8688) (width 0.3048) (layer "F.Cu") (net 5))
 (segment (start 195.5673 75.6158) (end 193.3067 75.6158) (width 0.3048) (layer "F.Cu") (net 5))
 (segment (start 198.0884 73.0947) (end 195.5673 75.6158) (width 0.3048) (layer "F.Cu") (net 5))
 (segment (start 202.0884 73.6417) (end 204.0171 75.5704) (width 0.3048) (layer "F.Cu") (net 11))
 (segment (start 202.0884 70.2056) (end 202.0884 73.6417) (width 0.3048) (layer "F.Cu") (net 11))
 (segment (start 204.0901 75.6434) (end 204.0171 75.5704) (width 0.3048) (layer "F.Cu") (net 11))
 (segment (start 208.7401 75.6434) (end 204.0901 75.6434) (width 0.3048) (layer "F.Cu") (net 11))
 (segment (start 200.9399 79.5308) (end 200.6097 79.861) (width 0.3048) (layer "F.Cu") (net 12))
 (segment (start 201.2884 69.9516) (end 201.2884 79.861) (width 0.3048) (layer "F.Cu") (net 12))
 (segment (start 205.5495 78.1812) (end 208.7379 78.1812) (width 0.3048) (layer "F.Cu") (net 12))
 (segment (start 204.1999 79.5308) (end 200.9399 79.5308) (width 0.3048) (layer "F.Cu") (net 12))
 (segment (start 204.1999 79.5308) (end 205.5495 78.1812) (width 0.3048) (layer "F.Cu") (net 12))
 (segment (start 201.2884 79.861) (end 200.6097 79.861) (width 0.3048) (layer "F.Cu") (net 12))
 (segment (start 208.7379 78.1812) (end 208.7401 78.1834) (width 0.3048) (layer "F.Cu") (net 12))
 (segment (start 207.6171 72.3704) (end 209.9171 72.3704) (width 0.3048) (layer "F.Cu") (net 13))
 (segment (start 211.4171 80.7174) (end 208.7401 80.7174) (width 0.3048) (layer "F.Cu") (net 13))
 (segment (start 205.9171 68.586) (end 205.9171 70.6704) (width 0.3048) (layer "F.Cu") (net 13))
 (segment (start 203.708 68.586) (end 205.9171 68.586) (width 0.3048) (layer "F.Cu") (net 13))
 (segment (start 209.9171 72.3704) (end 211.4171 73.8704) (width 0.3048) (layer "F.Cu") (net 13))
 (segment (start 208.7401 80.7174) (end 208.7401 80.7234) (width 0.3048) (layer "F.Cu") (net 13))
 (segment (start 211.4171 73.8704) (end 211.4171 80.7174) (width 0.3048) (layer "F.Cu") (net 13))
 (segment (start 214.511203 80.7174) (end 211.4171 80.7174) (width 0.3048) (layer "F.Cu") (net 13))
 (segment (start 205.9171 70.6704) (end 207.6171 72.3704) (width 0.3048) (layer "F.Cu") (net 13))
 (segment (start 195.1228 64.586) (end 191.0399 64.586) (width 0.3048) (layer "F.Cu") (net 1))
 (segment (start 214.5432 65.3933) (end 214.5432 72.2427) (width 0.3048) (layer "F.Cu") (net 1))
 (segment (start 203.454 65.386) (end 207.981 65.386) (width 0.3048) (layer "F.Cu") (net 1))
 (segment (start 200.1139 65.3796) (end 203.4476 65.3796) (width 0.3048) (layer "F.Cu") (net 1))
 (segment (start 211.536 65.3663) (end 211.536 65.3933) (width 0.3048) (layer "F.Cu") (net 1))
 (segment (start 182.6387 59.2762) (end 182.4609 59.0984) (width 0.3048) (layer "F.Cu") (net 1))
 (segment (start 207.981 65.386) (end 207.981 65.3663) (width 0.3048) (layer "F.Cu") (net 1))
 (segment (start 183.0377 58.5216) (end 183.0147 58.4986) (width 0.3048) (layer "F.Cu") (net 1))
 (segment (start 183.0377 58.5216) (end 182.4609 59.0984) (width 0.3048) (layer "F.Cu") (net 1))
 (segment (start 195.1228 66.1924) (end 195.1228 66.186) (width 0.3048) (layer "F.Cu") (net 1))
 (segment (start 197.4215 48.7172) (end 192.4177 43.7134) (width 0.3048) (layer "F.Cu") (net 1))
 (segment (start 181.8161 63.0664) (end 181.8304 63.0664) (width 0.3048) (layer "F.Cu") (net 1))
 (segment (start 191.0399 64.586) (end 190.8937 64.4398) (width 0.3048) (layer "F.Cu") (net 1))
 (segment (start 185.2295 58.5216) (end 183.0377 58.5216) (width 0.3048) (layer "F.Cu") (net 1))
 (segment (start 213.6145 61.1432) (end 213.5729 61.1016) (width 0.3048) (layer "F.Cu") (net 1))
 (segment (start 181.8161 61.5032) (end 182.6387 60.6806) (width 0.3048) (layer "F.Cu") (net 1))
 (segment (start 207.981 65.3663) (end 211.536 65.3663) (width 0.3048) (layer "F.Cu") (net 1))
 (segment (start 191.9605 66.1924) (end 190.8937 65.1256) (width 0.3048) (layer "F.Cu") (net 1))
 (segment (start 214.5432 65.3933) (end 214.5432 63.2481) (width 0.3048) (layer "F.Cu") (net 1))
 (segment (start 189.6237 58.5216) (end 185.2295 58.5216) (width 0.3048) (layer "F.Cu") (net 1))
 (segment (start 190.8937 59.7916) (end 189.6237 58.5216) (width 0.3048) (layer "F.Cu") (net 1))
 (segment (start 182.6387 60.6806) (end 182.6387 59.2762) (width 0.3048) (layer "F.Cu") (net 1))
 (segment (start 184.4167 49.4792) (end 184.4167 43.7134) (width 0.3048) (layer "F.Cu") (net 1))
 (segment (start 203.4476 65.3796) (end 203.454 65.386) (width 0.3048) (layer "F.Cu") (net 1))
 (segment (start 199.3203 64.586) (end 200.1139 65.3796) (width 0.3048) (layer "F.Cu") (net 1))
 (segment (start 214.5432 63.2481) (end 213.6267 62.3316) (width 0.3048) (layer "F.Cu") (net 1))
 (segment (start 195.1228 64.586) (end 199.3203 64.586) (width 0.3048) (layer "F.Cu") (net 1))
 (segment (start 211.536 65.3933) (end 214.5432 65.3933) (width 0.3048) (layer "F.Cu") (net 1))
 (segment (start 195.1228 64.586) (end 192.9511 64.586) (width 0.3048) (layer "F.Cu") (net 1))
 (segment (start 191.9605 66.1924) (end 195.1228 66.1924) (width 0.3048) (layer "F.Cu") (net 1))
 (segment (start 213.5729 56.2992) (end 213.5729 51.1948) (width 0.3048) (layer "F.Cu") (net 1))
 (segment (start 185.2295 50.292) (end 185.2295 58.5216) (width 0.3048) (layer "F.Cu") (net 1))
 (segment (start 201.0991 48.7172) (end 197.4215 48.7172) (width 0.3048) (layer "F.Cu") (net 1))
 (segment (start 213.6267 62.3316) (end 213.6267 61.1554) (width 0.3048) (layer "F.Cu") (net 1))
 (segment (start 213.5729 61.1016) (end 213.5729 56.2992) (width 0.3048) (layer "F.Cu") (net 1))
 (segment (start 190.8937 64.4398) (end 190.8937 59.7916) (width 0.3048) (layer "F.Cu") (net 1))
 (segment (start 184.4167 43.7134) (end 192.4177 43.7134) (width 0.3048) (layer "F.Cu") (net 1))
 (segment (start 190.8937 65.1256) (end 190.8937 64.4398) (width 0.3048) (layer "F.Cu") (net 1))
 (segment (start 213.6267 61.1554) (end 213.6145 61.1432) (width 0.3048) (layer "F.Cu") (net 1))
 (segment (start 181.8161 63.0664) (end 181.8161 61.5032) (width 0.3048) (layer "F.Cu") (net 1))
 (segment (start 181.8304 63.0664) (end 181.8304 72.4104) (width 0.3048) (layer "F.Cu") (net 1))
 (segment (start 185.2295 50.292) (end 184.4167 49.4792) (width 0.3048) (layer "F.Cu") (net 1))
 (segment (start 201.0991 46.392) (end 201.0991 48.7172) (width 0.3048) (layer "F.Cu") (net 1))
 (segment (start 174.5011 37.0036) (end 224.5011 37.0036) (width 0.1) (layer "B.Cu") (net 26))
 (segment (start 224.5011 87.0036) (end 174.5011 87.0036) (width 0.1) (layer "B.Cu") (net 26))
 (segment (start 174.5011 87.0036) (end 174.5011 37.0036) (width 0.1) (layer "B.Cu") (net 26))
 (segment (start 224.5011 37.0036) (end 224.5011 87.0036) (width 0.1) (layer "B.Cu") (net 26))
 (segment (start 182.9963 42.7228) (end 182.9963 46.3389) (width 0.3048) (layer "F.Cu") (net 10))
 (segment (start 216.3669 61.1016) (end 216.3669 56.2992) (width 0.3048) (layer "F.Cu") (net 10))
 (segment (start 182.9963 55.6986) (end 182.9963 46.3389) (width 0.3048) (layer "F.Cu") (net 10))
 (segment (start 211.509 68.1663) (end 211.536 68.1933) (width 0.3048) (layer "F.Cu") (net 10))
 (segment (start 216.3669 56.2992) (end 216.3669 51.1948) (width 0.3048) (layer "F.Cu") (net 10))
 (segment (start 183.0147 55.6986) (end 182.9963 55.6986) (width 0.3048) (layer "F.Cu") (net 10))
 (segment (start 198.5591 42.7228) (end 218.7067 42.7228) (width 0.3048) (layer "F.Cu") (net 10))
 (segment (start 216.4085 61.1432) (end 216.4085 73.66) (width 0.3048) (layer "F.Cu") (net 10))
 (segment (start 203.454 67.786) (end 205.8035 67.786) (width 0.3048) (layer "F.Cu") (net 10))
 (segment (start 207.981 67.786) (end 207.981 68.1663) (width 0.3048) (layer "F.Cu") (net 10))
 (segment (start 199.5043 67.7672) (end 203.4352 67.7672) (width 0.3048) (layer "F.Cu") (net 10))
 (segment (start 195.1228 65.386) (end 197.1231 65.386) (width 0.3048) (layer "F.Cu") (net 10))
 (segment (start 203.4352 67.7672) (end 203.454 67.786) (width 0.3048) (layer "F.Cu") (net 10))
 (segment (start 216.4085 61.1432) (end 216.3669 61.1016) (width 0.3048) (layer "F.Cu") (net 10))
 (segment (start 207.981 68.1663) (end 211.509 68.1663) (width 0.3048) (layer "F.Cu") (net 10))
 (segment (start 211.536 72.4329) (end 211.536 68.1933) (width 0.3048) (layer "F.Cu") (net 10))
 (segment (start 218.7067 48.26) (end 218.7067 42.7228) (width 0.3048) (layer "F.Cu") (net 10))
 (segment (start 203.454 66.186) (end 205.8035 66.186) (width 0.3048) (layer "F.Cu") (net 10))
 (segment (start 205.8035 66.186) (end 205.8035 67.786) (width 0.3048) (layer "F.Cu") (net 10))
 (segment (start 205.8035 67.786) (end 207.981 67.786) (width 0.3048) (layer "F.Cu") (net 10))
 (segment (start 197.1231 65.386) (end 198.7231 66.986) (width 0.3048) (layer "F.Cu") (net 10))
 (segment (start 195.1228 66.986) (end 198.7231 66.986) (width 0.3048) (layer "F.Cu") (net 10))
 (segment (start 216.3669 50.5998) (end 218.7067 48.26) (width 0.3048) (layer "F.Cu") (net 10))
 (segment (start 216.3669 51.1948) (end 216.3669 50.5998) (width 0.3048) (layer "F.Cu") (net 10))
 (segment (start 198.5591 46.392) (end 198.5591 42.7228) (width 0.3048) (layer "F.Cu") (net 10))
 (segment (start 198.7231 66.986) (end 199.5043 67.7672) (width 0.3048) (layer "F.Cu") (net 10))
 (segment (start 216.4085 73.66) (end 212.7631 73.66) (width 0.3048) (layer "F.Cu") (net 10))
 (segment (start 212.7631 73.66) (end 211.536 72.4329) (width 0.3048) (layer "F.Cu") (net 10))
 (segment (start 198.5591 42.7228) (end 182.9963 42.7228) (width 0.3048) (layer "F.Cu") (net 10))
 (segment (start 198.8884 73.7171) (end 195.8213 76.7842) (width 0.3048) (layer "F.Cu") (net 6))
 (segment (start 194.5767 76.7842) (end 193.0273 78.3336) (width 0.3048) (layer "F.Cu") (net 6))
 (segment (start 195.8213 76.7842) (end 194.5767 76.7842) (width 0.3048) (layer "F.Cu") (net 6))
 (segment (start 193.0273 79.8314) (end 192.9899 79.8688) (width 0.3048) (layer "F.Cu") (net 6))
 (segment (start 198.8884 69.9516) (end 198.8884 73.7171) (width 0.3048) (layer "F.Cu") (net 6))
 (segment (start 193.0273 78.3336) (end 193.0273 79.8314) (width 0.3048) (layer "F.Cu") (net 6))
 (segment (start 209.1055 61.6712) (end 209.1055 54.6804) (width 0.3048) (layer "F.Cu") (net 20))
 (segment (start 206.9907 63.786) (end 209.1055 61.6712) (width 0.3048) (layer "F.Cu") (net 20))
 (segment (start 209.1055 54.6804) (end 209.1171 54.6688) (width 0.3048) (layer "F.Cu") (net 20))
 (segment (start 203.454 63.786) (end 206.9907 63.786) (width 0.3048) (layer "F.Cu") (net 20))
 (segment (start 206.1143 62.986) (end 206.5909 62.5094) (width 0.3048) (layer "F.Cu") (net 16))
 (segment (start 206.5909 62.5094) (end 206.5909 54.6774) (width 0.3048) (layer "F.Cu") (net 16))
 (segment (start 203.708 62.986) (end 206.1143 62.986) (width 0.3048) (layer "F.Cu") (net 16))
 (segment (start 206.5909 54.6774) (end 206.5823 54.6688) (width 0.3048) (layer "F.Cu") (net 16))
 (segment (start 202.0884 61.3664) (end 202.0884 56.6279) (width 0.3048) (layer "F.Cu") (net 23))
 (segment (start 202.0884 56.6279) (end 204.0475 54.6688) (width 0.3048) (layer "F.Cu") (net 23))
 (segment (start 194.8688 61.4553) (end 188.5823 55.1688) (width 0.3048) (layer "F.Cu") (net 21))
 (segment (start 188.5823 55.1688) (end 187.989393 55.1688) (width 0.3048) (layer "F.Cu") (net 21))
 (segment (start 194.8688 62.986) (end 194.8688 61.4553) (width 0.3048) (layer "F.Cu") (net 21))
 (segment (start 187.989393 55.1688) (end 187.877106 55.056513) (width 0.3048) (layer "F.Cu") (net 21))
 (segment (start 199.6884 74.4919) (end 195.6689 78.5114) (width 0.3048) (layer "F.Cu") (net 22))
 (segment (start 199.6884 69.9516) (end 199.6884 74.4919) (width 0.3048) (layer "F.Cu") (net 22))
 (segment (start 195.6689 79.737775) (end 195.528915 79.87776) (width 0.3048) (layer "F.Cu") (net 22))
 (segment (start 195.6689 78.5114) (end 195.6689 79.737775) (width 0.3048) (layer "F.Cu") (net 22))
 (segment (start 198.069878 78.677179) (end 198.069878 79.87441) (width 0.3048) (layer "F.Cu") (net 14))
 (segment (start 200.4884 69.9516) (end 200.4884 75.8763) (width 0.3048) (layer "F.Cu") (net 14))
 (segment (start 198.0311 78.3336) (end 198.0311 78.6384) (width 0.3048) (layer "F.Cu") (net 14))
 (segment (start 200.4884 75.8763) (end 198.0311 78.3336) (width 0.3048) (layer "F.Cu") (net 14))
 (segment (start 198.0311 78.6384) (end 198.069878 78.677179) (width 0.3048) (layer "F.Cu") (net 14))
 (segment (start 197.2183 52.0947) (end 197.1803 52.0567) (width 0.3048) (layer "F.Cu") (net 24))
 (segment (start 197.2183 54.864) (end 197.2183 52.0947) (width 0.3048) (layer "F.Cu") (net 24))
 (segment (start 198.0884 61.6204) (end 198.0884 55.7341) (width 0.3048) (layer "F.Cu") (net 24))
 (segment (start 198.0884 55.7341) (end 197.2183 54.864) (width 0.3048) (layer "F.Cu") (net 24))
 (segment (start 194.3735 52.0695) (end 194.3863 52.0567) (width 0.3048) (layer "F.Cu") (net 25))
 (segment (start 197.2884 61.6204) (end 197.2884 57.2455) (width 0.3048) (layer "F.Cu") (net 25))
 (segment (start 194.3735 54.3306) (end 194.3735 52.0695) (width 0.3048) (layer "F.Cu") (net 25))
 (segment (start 197.2884 57.2455) (end 194.3735 54.3306) (width 0.3048) (layer "F.Cu") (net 25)))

